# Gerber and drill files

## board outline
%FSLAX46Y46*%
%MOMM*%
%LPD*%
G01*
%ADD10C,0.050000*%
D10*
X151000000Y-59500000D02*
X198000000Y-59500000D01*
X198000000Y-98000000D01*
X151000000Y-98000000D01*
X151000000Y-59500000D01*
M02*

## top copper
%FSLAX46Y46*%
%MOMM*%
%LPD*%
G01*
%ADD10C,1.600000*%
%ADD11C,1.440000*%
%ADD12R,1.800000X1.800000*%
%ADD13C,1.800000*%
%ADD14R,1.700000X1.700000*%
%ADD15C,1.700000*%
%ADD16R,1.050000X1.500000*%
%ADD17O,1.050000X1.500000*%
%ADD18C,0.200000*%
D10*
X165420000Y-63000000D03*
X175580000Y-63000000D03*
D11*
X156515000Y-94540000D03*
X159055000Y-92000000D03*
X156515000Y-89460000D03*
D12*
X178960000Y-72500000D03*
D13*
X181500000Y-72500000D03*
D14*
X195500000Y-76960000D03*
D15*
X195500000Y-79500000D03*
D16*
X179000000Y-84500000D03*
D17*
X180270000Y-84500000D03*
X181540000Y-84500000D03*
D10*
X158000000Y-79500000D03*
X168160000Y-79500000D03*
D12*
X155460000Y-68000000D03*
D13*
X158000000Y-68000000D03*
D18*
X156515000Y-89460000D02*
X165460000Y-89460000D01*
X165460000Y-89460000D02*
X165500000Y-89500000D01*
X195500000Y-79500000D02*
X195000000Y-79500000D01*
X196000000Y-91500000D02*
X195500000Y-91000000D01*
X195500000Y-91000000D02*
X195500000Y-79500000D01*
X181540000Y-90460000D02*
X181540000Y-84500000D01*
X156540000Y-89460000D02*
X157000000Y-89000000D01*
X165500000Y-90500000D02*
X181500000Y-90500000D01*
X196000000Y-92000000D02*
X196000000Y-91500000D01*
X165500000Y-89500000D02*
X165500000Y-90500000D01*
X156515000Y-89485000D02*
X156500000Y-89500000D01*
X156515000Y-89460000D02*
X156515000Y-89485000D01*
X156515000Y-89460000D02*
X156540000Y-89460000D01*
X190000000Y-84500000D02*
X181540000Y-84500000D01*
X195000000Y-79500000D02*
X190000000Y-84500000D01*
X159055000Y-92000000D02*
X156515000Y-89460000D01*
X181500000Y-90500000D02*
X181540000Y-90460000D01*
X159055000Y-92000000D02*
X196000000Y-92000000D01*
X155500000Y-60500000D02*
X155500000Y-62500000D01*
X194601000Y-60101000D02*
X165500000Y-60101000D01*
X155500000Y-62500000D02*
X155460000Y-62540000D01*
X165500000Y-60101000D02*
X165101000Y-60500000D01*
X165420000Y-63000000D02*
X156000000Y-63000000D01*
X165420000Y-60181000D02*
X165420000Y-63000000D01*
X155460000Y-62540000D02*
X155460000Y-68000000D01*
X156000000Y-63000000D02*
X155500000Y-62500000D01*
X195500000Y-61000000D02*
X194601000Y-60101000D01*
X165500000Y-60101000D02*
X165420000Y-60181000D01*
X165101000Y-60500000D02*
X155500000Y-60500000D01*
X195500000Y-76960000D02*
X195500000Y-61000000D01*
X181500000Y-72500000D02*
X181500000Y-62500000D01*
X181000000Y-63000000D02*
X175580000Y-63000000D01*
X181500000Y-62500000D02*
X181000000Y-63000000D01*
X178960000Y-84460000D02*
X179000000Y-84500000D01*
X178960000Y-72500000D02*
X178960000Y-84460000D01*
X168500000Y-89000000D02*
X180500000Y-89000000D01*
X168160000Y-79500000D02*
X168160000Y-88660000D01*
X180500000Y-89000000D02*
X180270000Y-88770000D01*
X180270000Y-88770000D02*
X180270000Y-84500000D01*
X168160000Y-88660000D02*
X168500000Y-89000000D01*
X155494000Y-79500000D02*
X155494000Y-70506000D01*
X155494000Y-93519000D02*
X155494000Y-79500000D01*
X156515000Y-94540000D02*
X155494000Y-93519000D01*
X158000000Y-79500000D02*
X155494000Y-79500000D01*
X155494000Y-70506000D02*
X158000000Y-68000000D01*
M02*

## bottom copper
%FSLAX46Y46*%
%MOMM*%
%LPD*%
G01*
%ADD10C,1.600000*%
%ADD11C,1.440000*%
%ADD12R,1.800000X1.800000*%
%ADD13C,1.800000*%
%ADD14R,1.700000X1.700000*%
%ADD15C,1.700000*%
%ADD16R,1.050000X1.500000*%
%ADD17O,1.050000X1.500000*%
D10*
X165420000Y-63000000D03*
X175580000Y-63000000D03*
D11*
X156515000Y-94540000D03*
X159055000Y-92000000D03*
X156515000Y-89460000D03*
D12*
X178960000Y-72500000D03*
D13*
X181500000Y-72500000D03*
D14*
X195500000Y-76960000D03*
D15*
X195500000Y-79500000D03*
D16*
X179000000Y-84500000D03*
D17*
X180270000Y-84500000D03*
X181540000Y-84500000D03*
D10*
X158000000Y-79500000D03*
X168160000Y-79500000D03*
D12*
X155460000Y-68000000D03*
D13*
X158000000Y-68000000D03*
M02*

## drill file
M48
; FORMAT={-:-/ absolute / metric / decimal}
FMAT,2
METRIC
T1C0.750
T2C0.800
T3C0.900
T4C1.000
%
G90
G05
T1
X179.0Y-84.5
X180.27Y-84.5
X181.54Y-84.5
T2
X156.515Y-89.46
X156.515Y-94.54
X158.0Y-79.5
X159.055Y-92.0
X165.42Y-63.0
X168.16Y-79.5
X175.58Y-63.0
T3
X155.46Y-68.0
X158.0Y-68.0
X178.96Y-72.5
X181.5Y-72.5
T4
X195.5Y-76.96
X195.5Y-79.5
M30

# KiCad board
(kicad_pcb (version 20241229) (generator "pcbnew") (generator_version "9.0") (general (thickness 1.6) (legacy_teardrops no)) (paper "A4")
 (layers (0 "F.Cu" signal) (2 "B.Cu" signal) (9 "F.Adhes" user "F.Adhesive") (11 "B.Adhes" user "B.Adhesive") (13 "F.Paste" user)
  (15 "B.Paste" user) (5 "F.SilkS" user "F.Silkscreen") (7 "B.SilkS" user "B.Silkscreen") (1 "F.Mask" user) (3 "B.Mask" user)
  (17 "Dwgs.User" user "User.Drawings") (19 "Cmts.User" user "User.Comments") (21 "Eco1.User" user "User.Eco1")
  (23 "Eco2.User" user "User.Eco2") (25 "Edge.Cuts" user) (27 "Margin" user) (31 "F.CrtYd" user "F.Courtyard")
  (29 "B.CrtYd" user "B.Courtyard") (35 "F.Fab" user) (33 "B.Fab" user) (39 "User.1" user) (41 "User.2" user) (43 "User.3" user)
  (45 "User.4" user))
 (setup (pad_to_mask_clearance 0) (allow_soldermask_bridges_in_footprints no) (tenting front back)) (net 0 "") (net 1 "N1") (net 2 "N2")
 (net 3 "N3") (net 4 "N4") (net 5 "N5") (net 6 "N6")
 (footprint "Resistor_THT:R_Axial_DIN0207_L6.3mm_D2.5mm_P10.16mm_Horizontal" (layer "F.Cu") (at 165.42 63)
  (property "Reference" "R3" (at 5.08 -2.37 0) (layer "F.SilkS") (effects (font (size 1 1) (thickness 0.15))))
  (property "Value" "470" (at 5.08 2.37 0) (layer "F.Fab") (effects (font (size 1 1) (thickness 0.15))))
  (pad "1" thru_hole circle (at 0 0) (size 1.6 1.6) (drill 0.8) (layers "*.Cu" "*.Mask") (remove_unused_layers no) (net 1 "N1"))
  (pad "2" thru_hole circle (at 10.16 0) (size 1.6 1.6) (drill 0.8) (layers "*.Cu" "*.Mask") (remove_unused_layers no) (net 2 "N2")))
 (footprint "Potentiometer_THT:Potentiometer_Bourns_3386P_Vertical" (layer "F.Cu") (at 156.515 94.54)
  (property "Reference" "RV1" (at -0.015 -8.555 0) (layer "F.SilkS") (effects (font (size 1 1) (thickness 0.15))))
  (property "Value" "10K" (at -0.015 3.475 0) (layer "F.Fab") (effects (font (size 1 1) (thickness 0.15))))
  (pad "1" thru_hole circle (at 0 0) (size 1.44 1.44) (drill 0.8) (layers "*.Cu" "*.Mask") (remove_unused_layers no) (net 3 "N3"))
  (pad "2" thru_hole circle (at 2.54 -2.54) (size 1.44 1.44) (drill 0.8) (layers "*.Cu" "*.Mask") (remove_unused_layers no) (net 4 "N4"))
  (pad "3" thru_hole circle (at 0 -5.08) (size 1.44 1.44) (drill 0.8) (layers "*.Cu" "*.Mask") (remove_unused_layers no) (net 4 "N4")))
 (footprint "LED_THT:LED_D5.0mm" (layer "F.Cu") (at 178.96 72.5)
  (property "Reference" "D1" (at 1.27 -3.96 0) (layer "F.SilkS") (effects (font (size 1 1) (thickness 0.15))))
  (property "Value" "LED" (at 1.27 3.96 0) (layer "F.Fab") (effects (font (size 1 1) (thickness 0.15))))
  (pad "1" thru_hole rect (at 0 0) (size 1.8 1.8) (drill 0.9) (layers "*.Cu" "*.Mask") (remove_unused_layers no) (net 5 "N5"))
  (pad "2" thru_hole circle (at 2.54 0) (size 1.8 1.8) (drill 0.9) (layers "*.Cu" "*.Mask") (remove_unused_layers no) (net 2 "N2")))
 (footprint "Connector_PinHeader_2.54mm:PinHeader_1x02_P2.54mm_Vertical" (layer "F.Cu") (at 195.5 76.96)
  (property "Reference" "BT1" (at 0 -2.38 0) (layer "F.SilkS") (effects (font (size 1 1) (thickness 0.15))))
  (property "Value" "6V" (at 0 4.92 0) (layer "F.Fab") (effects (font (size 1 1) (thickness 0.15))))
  (pad "1" thru_hole rect (at 0 0) (size 1.7 1.7) (drill 1) (layers "*.Cu" "*.Mask") (remove_unused_layers no) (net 1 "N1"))
  (pad "2" thru_hole circle (at 0 2.54) (size 1.7 1.7) (drill 1) (layers "*.Cu" "*.Mask") (remove_unused_layers no) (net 4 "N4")))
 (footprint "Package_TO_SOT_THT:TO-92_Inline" (layer "F.Cu") (at 179 84.5)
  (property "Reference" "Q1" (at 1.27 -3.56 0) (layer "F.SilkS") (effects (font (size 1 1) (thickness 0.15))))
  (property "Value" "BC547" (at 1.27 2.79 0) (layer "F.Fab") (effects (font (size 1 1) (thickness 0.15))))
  (pad "1" thru_hole rect (at 0 0) (size 1.05 1.5) (drill 0.75) (layers "*.Cu" "*.Mask") (remove_unused_layers no) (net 5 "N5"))
  (pad "2" thru_hole oval (at 1.27 0) (size 1.05 1.5) (drill 0.75) (layers "*.Cu" "*.Mask") (remove_unused_layers no) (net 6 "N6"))
  (pad "3" thru_hole oval (at 2.54 0) (size 1.05 1.5) (drill 0.75) (layers "*.Cu" "*.Mask") (remove_unused_layers no) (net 4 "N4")))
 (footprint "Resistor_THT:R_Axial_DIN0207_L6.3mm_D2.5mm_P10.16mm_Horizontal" (layer "F.Cu") (at 158 79.5)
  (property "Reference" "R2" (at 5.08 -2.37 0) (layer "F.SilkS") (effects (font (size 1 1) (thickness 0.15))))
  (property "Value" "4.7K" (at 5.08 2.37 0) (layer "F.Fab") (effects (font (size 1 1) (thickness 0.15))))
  (pad "1" thru_hole circle (at 0 0) (size 1.6 1.6) (drill 0.8) (layers "*.Cu" "*.Mask") (remove_unused_layers no) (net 3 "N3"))
  (pad "2" thru_hole circle (at 10.16 0) (size 1.6 1.6) (drill 0.8) (layers "*.Cu" "*.Mask") (remove_unused_layers no) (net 6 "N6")))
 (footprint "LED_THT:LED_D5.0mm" (layer "F.Cu") (at 155.46 68)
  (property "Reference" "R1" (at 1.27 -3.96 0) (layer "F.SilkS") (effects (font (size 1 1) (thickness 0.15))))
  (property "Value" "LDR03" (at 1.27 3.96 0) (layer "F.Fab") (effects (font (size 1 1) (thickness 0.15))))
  (pad "1" thru_hole rect (at 0 0) (size 1.8 1.8) (drill 0.9) (layers "*.Cu" "*.Mask") (remove_unused_layers no) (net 1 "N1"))
  (pad "2" thru_hole circle (at 2.54 0) (size 1.8 1.8) (drill 0.9) (layers "*.Cu" "*.Mask") (remove_unused_layers no) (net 3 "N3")))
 (gr_rect (start 151 59.5) (end 198 98) (stroke (width 0.05) (type default)) (fill no) (layer "Edge.Cuts"))
 (segment (start 156.515 89.46) (end 165.46 89.46) (width 0.2) (layer "F.Cu") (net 4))
 (segment (start 165.46 89.46) (end 165.5 89.5) (width 0.2) (layer "F.Cu") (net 4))
 (segment (start 195.5 79.5) (end 195 79.5) (width 0.2) (layer "F.Cu") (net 4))
 (segment (start 196 91.5) (end 195.5 91) (width 0.2) (layer "F.Cu") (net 4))
 (segment (start 195.5 91) (end 195.5 79.5) (width 0.2) (layer "F.Cu") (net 4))
 (segment (start 181.54 90.46) (end 181.54 84.5) (width 0.2) (layer "F.Cu") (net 4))
 (segment (start 156.54 89.46) (end 157 89) (width 0.2) (layer "F.Cu") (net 4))
 (segment (start 165.5 90.5) (end 181.5 90.5) (width 0.2) (layer "F.Cu") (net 4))
 (segment (start 196 92) (end 196 91.5) (width 0.2) (layer "F.Cu") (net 4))
 (segment (start 165.5 89.5) (end 165.5 90.5) (width 0.2) (layer "F.Cu") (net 4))
 (segment (start 156.515 89.485) (end 156.5 89.5) (width 0.2) (layer "F.Cu") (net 4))
 (segment (start 156.515 89.46) (end 156.515 89.485) (width 0.2) (layer "F.Cu") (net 4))
 (segment (start 156.515 89.46) (end 156.54 89.46) (width 0.2) (layer "F.Cu") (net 4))
 (segment (start 190 84.5) (end 181.54 84.5) (width 0.2) (layer "F.Cu") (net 4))
 (segment (start 195 79.5) (end 190 84.5) (width 0.2) (layer "F.Cu") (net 4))
 (segment (start 159.055 92) (end 156.515 89.46) (width 0.2) (layer "F.Cu") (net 4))
 (segment (start 181.5 90.5) (end 181.54 90.46) (width 0.2) (layer "F.Cu") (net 4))
 (segment (start 159.055 92) (end 196 92) (width 0.2) (layer "F.Cu") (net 4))
 (segment (start 155.5 60.5) (end 155.5 62.5) (width 0.2) (layer "F.Cu") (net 1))
 (segment (start 194.601 60.101) (end 165.5 60.101) (width 0.2) (layer "F.Cu") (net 1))
 (segment (start 155.5 62.5) (end 155.46 62.54) (width 0.2) (layer "F.Cu") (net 1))
 (segment (start 165.5 60.101) (end 165.101 60.5) (width 0.2) (layer "F.Cu") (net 1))
 (segment (start 165.42 63) (end 156 63) (width 0.2) (layer "F.Cu") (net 1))
 (segment (start 165.42 60.181) (end 165.42 63) (width 0.2) (layer "F.Cu") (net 1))
 (segment (start 155.46 62.54) (end 155.46 68) (width 0.2) (layer "F.Cu") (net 1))
 (segment (start 156 63) (end 155.5 62.5) (width 0.2) (layer "F.Cu") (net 1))
 (segment (start 195.5 61) (end 194.601 60.101) (width 0.2) (layer "F.Cu") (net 1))
 (segment (start 165.5 60.101) (end 165.42 60.181) (width 0.2) (layer "F.Cu") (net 1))
 (segment (start 165.101 60.5) (end 155.5 60.5) (width 0.2) (layer "F.Cu") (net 1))
 (segment (start 195.5 76.96) (end 195.5 61) (width 0.2) (layer "F.Cu") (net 1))
 (segment (start 181.5 72.5) (end 181.5 62.5) (width 0.2) (layer "F.Cu") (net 2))
 (segment (start 181 63) (end 175.58 63) (width 0.2) (layer "F.Cu") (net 2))
 (segment (start 181.5 62.5) (end 181 63) (width 0.2) (layer "F.Cu") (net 2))
 (segment (start 178.96 84.46) (end 179 84.5) (width 0.2) (layer "F.Cu") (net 5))
 (segment (start 178.96 72.5) (end 178.96 84.46) (width 0.2) (layer "F.Cu") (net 5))
 (segment (start 168.5 89) (end 180.5 89) (width 0.2) (layer "F.Cu") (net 6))
 (segment (start 168.16 79.5) (end 168.16 88.66) (width 0.2) (layer "F.Cu") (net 6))
 (segment (start 180.5 89) (end 180.27 88.77) (width 0.2) (layer "F.Cu") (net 6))
 (segment (start 180.27 88.77) (end 180.27 84.5) (width 0.2) (layer "F.Cu") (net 6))
 (segment (start 168.16 88.66) (end 168.5 89) (width 0.2) (layer "F.Cu") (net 6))
 (segment (start 155.494 79.5) (end 155.494 70.506) (width 0.2) (layer "F.Cu") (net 3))
 (segment (start 155.494 93.519) (end 155.494 79.5) (width 0.2) (layer "F.Cu") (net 3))
 (segment (start 156.515 94.54) (end 155.494 93.519) (width 0.2) (layer "F.Cu") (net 3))
 (segment (start 158 79.5) (end 155.494 79.5) (width 0.2) (layer "F.Cu") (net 3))
 (segment (start 155.494 70.506) (end 158 68) (width 0.2) (layer "F.Cu") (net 3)))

